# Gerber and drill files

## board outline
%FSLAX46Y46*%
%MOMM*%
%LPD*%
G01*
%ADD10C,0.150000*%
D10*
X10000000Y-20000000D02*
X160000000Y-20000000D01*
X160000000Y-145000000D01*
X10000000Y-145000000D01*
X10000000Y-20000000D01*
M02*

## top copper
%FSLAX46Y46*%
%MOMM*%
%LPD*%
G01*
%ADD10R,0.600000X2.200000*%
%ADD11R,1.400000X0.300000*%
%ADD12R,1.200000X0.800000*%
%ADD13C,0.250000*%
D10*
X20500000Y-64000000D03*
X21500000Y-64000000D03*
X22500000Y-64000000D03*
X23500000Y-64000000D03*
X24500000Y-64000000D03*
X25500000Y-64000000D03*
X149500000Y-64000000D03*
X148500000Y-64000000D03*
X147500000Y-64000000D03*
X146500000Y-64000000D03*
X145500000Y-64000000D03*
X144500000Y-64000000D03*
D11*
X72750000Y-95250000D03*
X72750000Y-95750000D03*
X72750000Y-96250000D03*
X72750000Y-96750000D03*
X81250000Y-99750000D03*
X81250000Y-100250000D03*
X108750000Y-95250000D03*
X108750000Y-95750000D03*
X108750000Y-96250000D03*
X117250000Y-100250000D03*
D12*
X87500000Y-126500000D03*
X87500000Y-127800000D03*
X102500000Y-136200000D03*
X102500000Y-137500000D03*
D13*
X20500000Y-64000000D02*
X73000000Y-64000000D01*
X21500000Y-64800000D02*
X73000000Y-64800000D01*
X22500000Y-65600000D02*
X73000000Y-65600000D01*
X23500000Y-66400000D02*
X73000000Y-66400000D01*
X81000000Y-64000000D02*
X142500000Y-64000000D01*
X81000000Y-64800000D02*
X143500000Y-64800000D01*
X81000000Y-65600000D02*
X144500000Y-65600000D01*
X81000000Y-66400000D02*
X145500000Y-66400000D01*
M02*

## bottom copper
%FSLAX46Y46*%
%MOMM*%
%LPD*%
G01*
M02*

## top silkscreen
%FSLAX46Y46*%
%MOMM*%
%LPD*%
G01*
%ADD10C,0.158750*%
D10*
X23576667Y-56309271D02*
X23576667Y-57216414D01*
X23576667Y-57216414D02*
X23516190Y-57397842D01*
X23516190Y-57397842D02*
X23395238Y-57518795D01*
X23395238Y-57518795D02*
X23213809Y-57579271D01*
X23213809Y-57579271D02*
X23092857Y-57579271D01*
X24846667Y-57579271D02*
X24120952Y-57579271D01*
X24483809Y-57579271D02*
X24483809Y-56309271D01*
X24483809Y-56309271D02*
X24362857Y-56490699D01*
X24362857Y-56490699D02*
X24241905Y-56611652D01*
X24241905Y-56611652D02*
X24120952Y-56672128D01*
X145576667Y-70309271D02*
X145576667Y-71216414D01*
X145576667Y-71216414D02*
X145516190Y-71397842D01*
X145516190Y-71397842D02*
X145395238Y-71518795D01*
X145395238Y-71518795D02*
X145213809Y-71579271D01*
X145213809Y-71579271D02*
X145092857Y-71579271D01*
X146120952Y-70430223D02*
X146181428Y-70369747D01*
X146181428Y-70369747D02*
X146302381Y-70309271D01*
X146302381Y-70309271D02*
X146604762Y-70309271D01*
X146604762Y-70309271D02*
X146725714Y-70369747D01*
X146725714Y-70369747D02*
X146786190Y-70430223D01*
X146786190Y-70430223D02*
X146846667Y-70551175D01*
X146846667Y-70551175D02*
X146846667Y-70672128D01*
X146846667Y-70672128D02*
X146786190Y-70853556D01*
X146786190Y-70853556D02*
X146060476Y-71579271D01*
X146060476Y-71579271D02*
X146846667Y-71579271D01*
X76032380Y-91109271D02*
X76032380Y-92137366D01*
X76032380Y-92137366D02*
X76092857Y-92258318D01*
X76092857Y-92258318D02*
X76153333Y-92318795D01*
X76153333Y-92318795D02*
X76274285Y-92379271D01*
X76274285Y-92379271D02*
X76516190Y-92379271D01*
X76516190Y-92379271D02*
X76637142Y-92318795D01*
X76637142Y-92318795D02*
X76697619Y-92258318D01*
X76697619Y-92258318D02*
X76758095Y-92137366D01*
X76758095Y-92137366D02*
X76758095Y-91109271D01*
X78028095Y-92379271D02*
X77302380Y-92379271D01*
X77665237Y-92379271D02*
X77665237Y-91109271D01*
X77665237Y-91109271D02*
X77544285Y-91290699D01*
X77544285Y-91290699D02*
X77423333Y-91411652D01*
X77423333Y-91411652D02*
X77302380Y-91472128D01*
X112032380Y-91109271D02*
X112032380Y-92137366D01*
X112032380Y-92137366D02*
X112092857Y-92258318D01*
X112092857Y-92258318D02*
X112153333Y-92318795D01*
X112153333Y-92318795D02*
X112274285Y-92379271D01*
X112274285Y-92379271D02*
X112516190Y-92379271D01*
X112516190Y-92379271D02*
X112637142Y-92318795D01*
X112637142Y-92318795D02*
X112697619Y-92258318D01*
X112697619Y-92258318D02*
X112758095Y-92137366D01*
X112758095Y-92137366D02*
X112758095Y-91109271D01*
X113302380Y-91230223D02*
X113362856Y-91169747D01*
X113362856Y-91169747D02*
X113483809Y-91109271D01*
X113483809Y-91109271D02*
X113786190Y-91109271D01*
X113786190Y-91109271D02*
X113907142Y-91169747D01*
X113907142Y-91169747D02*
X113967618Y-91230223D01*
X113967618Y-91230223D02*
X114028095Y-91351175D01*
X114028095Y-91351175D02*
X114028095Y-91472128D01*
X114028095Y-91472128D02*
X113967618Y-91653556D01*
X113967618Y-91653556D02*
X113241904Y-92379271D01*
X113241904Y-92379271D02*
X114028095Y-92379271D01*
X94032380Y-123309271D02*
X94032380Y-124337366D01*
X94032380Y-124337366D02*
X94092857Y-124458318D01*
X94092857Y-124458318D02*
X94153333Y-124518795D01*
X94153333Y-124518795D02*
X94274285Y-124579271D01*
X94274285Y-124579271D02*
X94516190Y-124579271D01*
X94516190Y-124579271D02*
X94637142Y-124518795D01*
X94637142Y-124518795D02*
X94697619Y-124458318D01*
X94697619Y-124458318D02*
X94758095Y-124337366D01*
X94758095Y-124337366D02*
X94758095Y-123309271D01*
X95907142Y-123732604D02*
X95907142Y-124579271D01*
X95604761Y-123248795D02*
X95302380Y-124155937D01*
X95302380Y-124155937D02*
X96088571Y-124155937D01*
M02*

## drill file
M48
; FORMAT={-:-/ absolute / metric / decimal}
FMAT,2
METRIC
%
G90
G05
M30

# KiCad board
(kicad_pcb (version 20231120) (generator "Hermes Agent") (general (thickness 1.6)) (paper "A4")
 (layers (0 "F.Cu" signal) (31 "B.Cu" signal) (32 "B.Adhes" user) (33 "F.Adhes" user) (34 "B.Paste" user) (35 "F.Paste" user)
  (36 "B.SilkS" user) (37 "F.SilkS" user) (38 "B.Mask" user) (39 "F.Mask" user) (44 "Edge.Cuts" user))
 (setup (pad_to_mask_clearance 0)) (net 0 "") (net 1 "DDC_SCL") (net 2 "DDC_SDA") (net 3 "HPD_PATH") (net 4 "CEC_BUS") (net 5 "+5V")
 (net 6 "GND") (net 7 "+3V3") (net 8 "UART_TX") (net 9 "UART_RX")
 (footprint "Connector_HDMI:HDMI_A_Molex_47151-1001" (layer "F.Cu") (at 24 64) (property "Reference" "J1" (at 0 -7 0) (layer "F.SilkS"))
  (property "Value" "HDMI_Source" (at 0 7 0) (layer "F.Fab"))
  (pad "15" smd rect (at -3.5 0) (size 0.6 2.2) (layers "F.Cu" "F.Mask" "F.Paste") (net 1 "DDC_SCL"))
  (pad "16" smd rect (at -2.5 0) (size 0.6 2.2) (layers "F.Cu" "F.Mask" "F.Paste") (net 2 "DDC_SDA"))
  (pad "19" smd rect (at -1.5 0) (size 0.6 2.2) (layers "F.Cu" "F.Mask" "F.Paste") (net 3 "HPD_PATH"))
  (pad "13" smd rect (at -0.5 0) (size 0.6 2.2) (layers "F.Cu" "F.Mask" "F.Paste") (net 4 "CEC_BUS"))
  (pad "18" smd rect (at 0.5 0) (size 0.6 2.2) (layers "F.Cu" "F.Mask" "F.Paste") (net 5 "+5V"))
  (pad "17" smd rect (at 1.5 0) (size 0.6 2.2) (layers "F.Cu" "F.Mask" "F.Paste") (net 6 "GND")))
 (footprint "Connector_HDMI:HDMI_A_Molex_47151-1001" (layer "F.Cu") (at 146 64 180)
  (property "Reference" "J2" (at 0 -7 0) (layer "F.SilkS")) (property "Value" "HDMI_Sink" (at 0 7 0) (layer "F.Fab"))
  (pad "15" smd rect (at -3.5 0) (size 0.6 2.2) (layers "F.Cu" "F.Mask" "F.Paste") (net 1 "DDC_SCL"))
  (pad "16" smd rect (at -2.5 0) (size 0.6 2.2) (layers "F.Cu" "F.Mask" "F.Paste") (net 2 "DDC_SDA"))
  (pad "19" smd rect (at -1.5 0) (size 0.6 2.2) (layers "F.Cu" "F.Mask" "F.Paste") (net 3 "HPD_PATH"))
  (pad "13" smd rect (at -0.5 0) (size 0.6 2.2) (layers "F.Cu" "F.Mask" "F.Paste") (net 4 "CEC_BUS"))
  (pad "18" smd rect (at 0.5 0) (size 0.6 2.2) (layers "F.Cu" "F.Mask" "F.Paste") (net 5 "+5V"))
  (pad "17" smd rect (at 1.5 0) (size 0.6 2.2) (layers "F.Cu" "F.Mask" "F.Paste") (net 6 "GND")))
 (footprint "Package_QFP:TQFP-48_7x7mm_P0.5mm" (layer "F.Cu") (at 77 98) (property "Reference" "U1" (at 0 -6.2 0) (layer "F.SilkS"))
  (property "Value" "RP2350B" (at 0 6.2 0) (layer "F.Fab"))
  (pad "1" smd rect (at -4.25 -2.75) (size 1.4 0.3) (layers "F.Cu" "F.Mask" "F.Paste") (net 2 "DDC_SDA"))
  (pad "2" smd rect (at -4.25 -2.25) (size 1.4 0.3) (layers "F.Cu" "F.Mask" "F.Paste") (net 1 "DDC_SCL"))
  (pad "3" smd rect (at -4.25 -1.75) (size 1.4 0.3) (layers "F.Cu" "F.Mask" "F.Paste") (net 3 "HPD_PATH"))
  (pad "4" smd rect (at -4.25 -1.25) (size 1.4 0.3) (layers "F.Cu" "F.Mask" "F.Paste") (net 4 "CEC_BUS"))
  (pad "40" smd rect (at 4.25 1.75) (size 1.4 0.3) (layers "F.Cu" "F.Mask" "F.Paste") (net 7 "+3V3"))
  (pad "41" smd rect (at 4.25 2.25) (size 1.4 0.3) (layers "F.Cu" "F.Mask" "F.Paste") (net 6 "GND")))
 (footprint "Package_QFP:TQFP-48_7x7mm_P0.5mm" (layer "F.Cu") (at 113 98) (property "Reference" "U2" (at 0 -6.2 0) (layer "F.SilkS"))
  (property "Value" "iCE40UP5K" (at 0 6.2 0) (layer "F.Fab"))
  (pad "1" smd rect (at -4.25 -2.75) (size 1.4 0.3) (layers "F.Cu" "F.Mask" "F.Paste") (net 2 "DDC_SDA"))
  (pad "2" smd rect (at -4.25 -2.25) (size 1.4 0.3) (layers "F.Cu" "F.Mask" "F.Paste") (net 1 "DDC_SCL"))
  (pad "3" smd rect (at -4.25 -1.75) (size 1.4 0.3) (layers "F.Cu" "F.Mask" "F.Paste") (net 3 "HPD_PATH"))
  (pad "48" smd rect (at 4.25 2.25) (size 1.4 0.3) (layers "F.Cu" "F.Mask" "F.Paste") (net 6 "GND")))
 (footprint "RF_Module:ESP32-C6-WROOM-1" (layer "F.Cu") (at 95 132) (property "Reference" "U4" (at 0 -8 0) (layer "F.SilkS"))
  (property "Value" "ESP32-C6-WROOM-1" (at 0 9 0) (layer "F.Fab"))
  (pad "1" smd rect (at -7.5 -5.5) (size 1.2 0.8) (layers "F.Cu" "F.Mask" "F.Paste") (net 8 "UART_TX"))
  (pad "2" smd rect (at -7.5 -4.2) (size 1.2 0.8) (layers "F.Cu" "F.Mask" "F.Paste") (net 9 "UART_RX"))
  (pad "28" smd rect (at 7.5 4.2) (size 1.2 0.8) (layers "F.Cu" "F.Mask" "F.Paste") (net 7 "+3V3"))
  (pad "29" smd rect (at 7.5 5.5) (size 1.2 0.8) (layers "F.Cu" "F.Mask" "F.Paste") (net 6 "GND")))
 (gr_rect (start 10 20) (end 160 145) (stroke (width 0.15) (type default)) (fill none) (layer "Edge.Cuts"))
 (segment (start 20.5 64) (end 73 64) (width 0.25) (layer "F.Cu") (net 1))
 (segment (start 21.5 64.8) (end 73 64.8) (width 0.25) (layer "F.Cu") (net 2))
 (segment (start 22.5 65.6) (end 73 65.6) (width 0.25) (layer "F.Cu") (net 3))
 (segment (start 23.5 66.4) (end 73 66.4) (width 0.25) (layer "F.Cu") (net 4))
 (segment (start 81 64) (end 142.5 64) (width 0.25) (layer "F.Cu") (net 1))
 (segment (start 81 64.8) (end 143.5 64.8) (width 0.25) (layer "F.Cu") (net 2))
 (segment (start 81 65.6) (end 144.5 65.6) (width 0.25) (layer "F.Cu") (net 3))
 (segment (start 81 66.4) (end 145.5 66.4) (width 0.25) (layer "F.Cu") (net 4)))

